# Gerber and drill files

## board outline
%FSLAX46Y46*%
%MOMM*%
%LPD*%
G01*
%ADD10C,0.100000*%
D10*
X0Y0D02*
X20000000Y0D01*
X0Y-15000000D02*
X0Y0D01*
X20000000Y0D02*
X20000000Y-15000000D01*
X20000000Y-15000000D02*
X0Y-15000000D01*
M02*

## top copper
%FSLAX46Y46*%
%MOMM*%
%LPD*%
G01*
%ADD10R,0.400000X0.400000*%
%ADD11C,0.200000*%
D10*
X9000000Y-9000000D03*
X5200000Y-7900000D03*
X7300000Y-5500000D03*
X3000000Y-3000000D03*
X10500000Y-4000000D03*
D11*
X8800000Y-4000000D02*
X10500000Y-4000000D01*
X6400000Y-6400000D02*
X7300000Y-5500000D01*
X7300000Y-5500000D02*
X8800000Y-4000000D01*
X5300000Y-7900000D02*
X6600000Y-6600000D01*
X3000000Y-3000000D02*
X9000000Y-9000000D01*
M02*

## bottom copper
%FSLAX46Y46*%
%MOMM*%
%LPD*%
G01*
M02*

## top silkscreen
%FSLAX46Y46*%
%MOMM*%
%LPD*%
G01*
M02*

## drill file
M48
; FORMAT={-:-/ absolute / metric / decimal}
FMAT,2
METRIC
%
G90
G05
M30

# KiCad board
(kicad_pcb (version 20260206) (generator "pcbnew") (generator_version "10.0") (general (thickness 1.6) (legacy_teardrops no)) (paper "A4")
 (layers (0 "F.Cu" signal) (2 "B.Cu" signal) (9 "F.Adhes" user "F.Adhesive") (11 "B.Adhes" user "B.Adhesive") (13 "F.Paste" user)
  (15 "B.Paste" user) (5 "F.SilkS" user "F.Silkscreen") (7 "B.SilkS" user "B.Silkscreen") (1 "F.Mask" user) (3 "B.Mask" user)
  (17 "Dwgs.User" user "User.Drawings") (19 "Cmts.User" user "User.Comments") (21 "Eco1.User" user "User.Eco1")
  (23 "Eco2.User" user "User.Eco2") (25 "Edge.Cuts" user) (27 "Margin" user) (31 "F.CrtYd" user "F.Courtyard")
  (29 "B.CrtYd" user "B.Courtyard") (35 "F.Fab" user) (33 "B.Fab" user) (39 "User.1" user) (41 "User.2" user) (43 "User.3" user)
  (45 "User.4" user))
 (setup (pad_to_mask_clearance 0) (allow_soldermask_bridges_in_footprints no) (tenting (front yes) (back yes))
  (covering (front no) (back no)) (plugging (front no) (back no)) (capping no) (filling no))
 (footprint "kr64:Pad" (layer "F.Cu") (at 9 9)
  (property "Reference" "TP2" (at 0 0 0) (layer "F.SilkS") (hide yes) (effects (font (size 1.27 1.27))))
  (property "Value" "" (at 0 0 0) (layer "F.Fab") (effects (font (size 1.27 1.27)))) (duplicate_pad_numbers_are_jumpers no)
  (pad "1" smd rect (at 0 0) (size 0.4 0.4) (layers "F.Cu" "F.Mask" "F.Paste") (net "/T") (thermal_bridge_angle 45)))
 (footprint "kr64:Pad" (layer "F.Cu") (at 5.2 7.9)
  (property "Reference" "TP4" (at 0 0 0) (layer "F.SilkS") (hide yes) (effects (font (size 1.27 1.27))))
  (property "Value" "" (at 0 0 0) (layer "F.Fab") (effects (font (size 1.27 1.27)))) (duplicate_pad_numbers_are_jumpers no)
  (pad "1" smd rect (at 0 0) (size 0.4 0.4) (layers "F.Cu" "F.Mask" "F.Paste") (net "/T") (thermal_bridge_angle 45)))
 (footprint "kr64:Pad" (layer "F.Cu") (at 7.3 5.5)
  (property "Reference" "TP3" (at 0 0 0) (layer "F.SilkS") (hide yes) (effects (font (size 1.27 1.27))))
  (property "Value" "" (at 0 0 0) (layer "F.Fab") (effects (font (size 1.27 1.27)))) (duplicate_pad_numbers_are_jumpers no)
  (pad "1" smd rect (at 0 0) (size 0.4 0.4) (layers "F.Cu" "F.Mask" "F.Paste") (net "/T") (thermal_bridge_angle 45)))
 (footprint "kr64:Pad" (layer "F.Cu") (at 3 3)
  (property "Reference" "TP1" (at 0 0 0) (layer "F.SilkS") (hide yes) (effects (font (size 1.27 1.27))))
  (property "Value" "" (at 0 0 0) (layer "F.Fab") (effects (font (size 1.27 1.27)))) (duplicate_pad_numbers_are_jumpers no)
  (pad "1" smd rect (at 0 0) (size 0.4 0.4) (layers "F.Cu" "F.Mask" "F.Paste") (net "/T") (thermal_bridge_angle 45)))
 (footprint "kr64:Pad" (layer "F.Cu") (at 10.5 4)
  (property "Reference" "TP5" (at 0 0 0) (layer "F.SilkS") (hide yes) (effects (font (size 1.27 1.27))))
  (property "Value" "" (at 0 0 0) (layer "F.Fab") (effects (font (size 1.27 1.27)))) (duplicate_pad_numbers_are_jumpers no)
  (pad "1" smd rect (at 0 0) (size 0.4 0.4) (layers "F.Cu" "F.Mask" "F.Paste") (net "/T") (thermal_bridge_angle 45)))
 (gr_line (start 0 0) (end 20 0) (stroke (width 0.1) (type default)) (layer "Edge.Cuts"))
 (gr_line (start 0 15) (end 0 0) (stroke (width 0.1) (type default)) (layer "Edge.Cuts"))
 (gr_line (start 20 0) (end 20 15) (stroke (width 0.1) (type default)) (layer "Edge.Cuts"))
 (gr_line (start 20 15) (end 0 15) (stroke (width 0.1) (type default)) (layer "Edge.Cuts"))
 (segment (start 8.8 4) (end 10.5 4) (width 0.2) (layer "F.Cu") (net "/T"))
 (segment (start 6.4 6.4) (end 7.3 5.5) (width 0.2) (layer "F.Cu") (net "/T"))
 (segment (start 7.3 5.5) (end 8.8 4) (width 0.2) (layer "F.Cu") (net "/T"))
 (segment (start 5.3 7.9) (end 6.6 6.6) (width 0.2) (layer "F.Cu") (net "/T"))
 (segment (start 3 3) (end 9 9) (width 0.2) (layer "F.Cu") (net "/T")))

